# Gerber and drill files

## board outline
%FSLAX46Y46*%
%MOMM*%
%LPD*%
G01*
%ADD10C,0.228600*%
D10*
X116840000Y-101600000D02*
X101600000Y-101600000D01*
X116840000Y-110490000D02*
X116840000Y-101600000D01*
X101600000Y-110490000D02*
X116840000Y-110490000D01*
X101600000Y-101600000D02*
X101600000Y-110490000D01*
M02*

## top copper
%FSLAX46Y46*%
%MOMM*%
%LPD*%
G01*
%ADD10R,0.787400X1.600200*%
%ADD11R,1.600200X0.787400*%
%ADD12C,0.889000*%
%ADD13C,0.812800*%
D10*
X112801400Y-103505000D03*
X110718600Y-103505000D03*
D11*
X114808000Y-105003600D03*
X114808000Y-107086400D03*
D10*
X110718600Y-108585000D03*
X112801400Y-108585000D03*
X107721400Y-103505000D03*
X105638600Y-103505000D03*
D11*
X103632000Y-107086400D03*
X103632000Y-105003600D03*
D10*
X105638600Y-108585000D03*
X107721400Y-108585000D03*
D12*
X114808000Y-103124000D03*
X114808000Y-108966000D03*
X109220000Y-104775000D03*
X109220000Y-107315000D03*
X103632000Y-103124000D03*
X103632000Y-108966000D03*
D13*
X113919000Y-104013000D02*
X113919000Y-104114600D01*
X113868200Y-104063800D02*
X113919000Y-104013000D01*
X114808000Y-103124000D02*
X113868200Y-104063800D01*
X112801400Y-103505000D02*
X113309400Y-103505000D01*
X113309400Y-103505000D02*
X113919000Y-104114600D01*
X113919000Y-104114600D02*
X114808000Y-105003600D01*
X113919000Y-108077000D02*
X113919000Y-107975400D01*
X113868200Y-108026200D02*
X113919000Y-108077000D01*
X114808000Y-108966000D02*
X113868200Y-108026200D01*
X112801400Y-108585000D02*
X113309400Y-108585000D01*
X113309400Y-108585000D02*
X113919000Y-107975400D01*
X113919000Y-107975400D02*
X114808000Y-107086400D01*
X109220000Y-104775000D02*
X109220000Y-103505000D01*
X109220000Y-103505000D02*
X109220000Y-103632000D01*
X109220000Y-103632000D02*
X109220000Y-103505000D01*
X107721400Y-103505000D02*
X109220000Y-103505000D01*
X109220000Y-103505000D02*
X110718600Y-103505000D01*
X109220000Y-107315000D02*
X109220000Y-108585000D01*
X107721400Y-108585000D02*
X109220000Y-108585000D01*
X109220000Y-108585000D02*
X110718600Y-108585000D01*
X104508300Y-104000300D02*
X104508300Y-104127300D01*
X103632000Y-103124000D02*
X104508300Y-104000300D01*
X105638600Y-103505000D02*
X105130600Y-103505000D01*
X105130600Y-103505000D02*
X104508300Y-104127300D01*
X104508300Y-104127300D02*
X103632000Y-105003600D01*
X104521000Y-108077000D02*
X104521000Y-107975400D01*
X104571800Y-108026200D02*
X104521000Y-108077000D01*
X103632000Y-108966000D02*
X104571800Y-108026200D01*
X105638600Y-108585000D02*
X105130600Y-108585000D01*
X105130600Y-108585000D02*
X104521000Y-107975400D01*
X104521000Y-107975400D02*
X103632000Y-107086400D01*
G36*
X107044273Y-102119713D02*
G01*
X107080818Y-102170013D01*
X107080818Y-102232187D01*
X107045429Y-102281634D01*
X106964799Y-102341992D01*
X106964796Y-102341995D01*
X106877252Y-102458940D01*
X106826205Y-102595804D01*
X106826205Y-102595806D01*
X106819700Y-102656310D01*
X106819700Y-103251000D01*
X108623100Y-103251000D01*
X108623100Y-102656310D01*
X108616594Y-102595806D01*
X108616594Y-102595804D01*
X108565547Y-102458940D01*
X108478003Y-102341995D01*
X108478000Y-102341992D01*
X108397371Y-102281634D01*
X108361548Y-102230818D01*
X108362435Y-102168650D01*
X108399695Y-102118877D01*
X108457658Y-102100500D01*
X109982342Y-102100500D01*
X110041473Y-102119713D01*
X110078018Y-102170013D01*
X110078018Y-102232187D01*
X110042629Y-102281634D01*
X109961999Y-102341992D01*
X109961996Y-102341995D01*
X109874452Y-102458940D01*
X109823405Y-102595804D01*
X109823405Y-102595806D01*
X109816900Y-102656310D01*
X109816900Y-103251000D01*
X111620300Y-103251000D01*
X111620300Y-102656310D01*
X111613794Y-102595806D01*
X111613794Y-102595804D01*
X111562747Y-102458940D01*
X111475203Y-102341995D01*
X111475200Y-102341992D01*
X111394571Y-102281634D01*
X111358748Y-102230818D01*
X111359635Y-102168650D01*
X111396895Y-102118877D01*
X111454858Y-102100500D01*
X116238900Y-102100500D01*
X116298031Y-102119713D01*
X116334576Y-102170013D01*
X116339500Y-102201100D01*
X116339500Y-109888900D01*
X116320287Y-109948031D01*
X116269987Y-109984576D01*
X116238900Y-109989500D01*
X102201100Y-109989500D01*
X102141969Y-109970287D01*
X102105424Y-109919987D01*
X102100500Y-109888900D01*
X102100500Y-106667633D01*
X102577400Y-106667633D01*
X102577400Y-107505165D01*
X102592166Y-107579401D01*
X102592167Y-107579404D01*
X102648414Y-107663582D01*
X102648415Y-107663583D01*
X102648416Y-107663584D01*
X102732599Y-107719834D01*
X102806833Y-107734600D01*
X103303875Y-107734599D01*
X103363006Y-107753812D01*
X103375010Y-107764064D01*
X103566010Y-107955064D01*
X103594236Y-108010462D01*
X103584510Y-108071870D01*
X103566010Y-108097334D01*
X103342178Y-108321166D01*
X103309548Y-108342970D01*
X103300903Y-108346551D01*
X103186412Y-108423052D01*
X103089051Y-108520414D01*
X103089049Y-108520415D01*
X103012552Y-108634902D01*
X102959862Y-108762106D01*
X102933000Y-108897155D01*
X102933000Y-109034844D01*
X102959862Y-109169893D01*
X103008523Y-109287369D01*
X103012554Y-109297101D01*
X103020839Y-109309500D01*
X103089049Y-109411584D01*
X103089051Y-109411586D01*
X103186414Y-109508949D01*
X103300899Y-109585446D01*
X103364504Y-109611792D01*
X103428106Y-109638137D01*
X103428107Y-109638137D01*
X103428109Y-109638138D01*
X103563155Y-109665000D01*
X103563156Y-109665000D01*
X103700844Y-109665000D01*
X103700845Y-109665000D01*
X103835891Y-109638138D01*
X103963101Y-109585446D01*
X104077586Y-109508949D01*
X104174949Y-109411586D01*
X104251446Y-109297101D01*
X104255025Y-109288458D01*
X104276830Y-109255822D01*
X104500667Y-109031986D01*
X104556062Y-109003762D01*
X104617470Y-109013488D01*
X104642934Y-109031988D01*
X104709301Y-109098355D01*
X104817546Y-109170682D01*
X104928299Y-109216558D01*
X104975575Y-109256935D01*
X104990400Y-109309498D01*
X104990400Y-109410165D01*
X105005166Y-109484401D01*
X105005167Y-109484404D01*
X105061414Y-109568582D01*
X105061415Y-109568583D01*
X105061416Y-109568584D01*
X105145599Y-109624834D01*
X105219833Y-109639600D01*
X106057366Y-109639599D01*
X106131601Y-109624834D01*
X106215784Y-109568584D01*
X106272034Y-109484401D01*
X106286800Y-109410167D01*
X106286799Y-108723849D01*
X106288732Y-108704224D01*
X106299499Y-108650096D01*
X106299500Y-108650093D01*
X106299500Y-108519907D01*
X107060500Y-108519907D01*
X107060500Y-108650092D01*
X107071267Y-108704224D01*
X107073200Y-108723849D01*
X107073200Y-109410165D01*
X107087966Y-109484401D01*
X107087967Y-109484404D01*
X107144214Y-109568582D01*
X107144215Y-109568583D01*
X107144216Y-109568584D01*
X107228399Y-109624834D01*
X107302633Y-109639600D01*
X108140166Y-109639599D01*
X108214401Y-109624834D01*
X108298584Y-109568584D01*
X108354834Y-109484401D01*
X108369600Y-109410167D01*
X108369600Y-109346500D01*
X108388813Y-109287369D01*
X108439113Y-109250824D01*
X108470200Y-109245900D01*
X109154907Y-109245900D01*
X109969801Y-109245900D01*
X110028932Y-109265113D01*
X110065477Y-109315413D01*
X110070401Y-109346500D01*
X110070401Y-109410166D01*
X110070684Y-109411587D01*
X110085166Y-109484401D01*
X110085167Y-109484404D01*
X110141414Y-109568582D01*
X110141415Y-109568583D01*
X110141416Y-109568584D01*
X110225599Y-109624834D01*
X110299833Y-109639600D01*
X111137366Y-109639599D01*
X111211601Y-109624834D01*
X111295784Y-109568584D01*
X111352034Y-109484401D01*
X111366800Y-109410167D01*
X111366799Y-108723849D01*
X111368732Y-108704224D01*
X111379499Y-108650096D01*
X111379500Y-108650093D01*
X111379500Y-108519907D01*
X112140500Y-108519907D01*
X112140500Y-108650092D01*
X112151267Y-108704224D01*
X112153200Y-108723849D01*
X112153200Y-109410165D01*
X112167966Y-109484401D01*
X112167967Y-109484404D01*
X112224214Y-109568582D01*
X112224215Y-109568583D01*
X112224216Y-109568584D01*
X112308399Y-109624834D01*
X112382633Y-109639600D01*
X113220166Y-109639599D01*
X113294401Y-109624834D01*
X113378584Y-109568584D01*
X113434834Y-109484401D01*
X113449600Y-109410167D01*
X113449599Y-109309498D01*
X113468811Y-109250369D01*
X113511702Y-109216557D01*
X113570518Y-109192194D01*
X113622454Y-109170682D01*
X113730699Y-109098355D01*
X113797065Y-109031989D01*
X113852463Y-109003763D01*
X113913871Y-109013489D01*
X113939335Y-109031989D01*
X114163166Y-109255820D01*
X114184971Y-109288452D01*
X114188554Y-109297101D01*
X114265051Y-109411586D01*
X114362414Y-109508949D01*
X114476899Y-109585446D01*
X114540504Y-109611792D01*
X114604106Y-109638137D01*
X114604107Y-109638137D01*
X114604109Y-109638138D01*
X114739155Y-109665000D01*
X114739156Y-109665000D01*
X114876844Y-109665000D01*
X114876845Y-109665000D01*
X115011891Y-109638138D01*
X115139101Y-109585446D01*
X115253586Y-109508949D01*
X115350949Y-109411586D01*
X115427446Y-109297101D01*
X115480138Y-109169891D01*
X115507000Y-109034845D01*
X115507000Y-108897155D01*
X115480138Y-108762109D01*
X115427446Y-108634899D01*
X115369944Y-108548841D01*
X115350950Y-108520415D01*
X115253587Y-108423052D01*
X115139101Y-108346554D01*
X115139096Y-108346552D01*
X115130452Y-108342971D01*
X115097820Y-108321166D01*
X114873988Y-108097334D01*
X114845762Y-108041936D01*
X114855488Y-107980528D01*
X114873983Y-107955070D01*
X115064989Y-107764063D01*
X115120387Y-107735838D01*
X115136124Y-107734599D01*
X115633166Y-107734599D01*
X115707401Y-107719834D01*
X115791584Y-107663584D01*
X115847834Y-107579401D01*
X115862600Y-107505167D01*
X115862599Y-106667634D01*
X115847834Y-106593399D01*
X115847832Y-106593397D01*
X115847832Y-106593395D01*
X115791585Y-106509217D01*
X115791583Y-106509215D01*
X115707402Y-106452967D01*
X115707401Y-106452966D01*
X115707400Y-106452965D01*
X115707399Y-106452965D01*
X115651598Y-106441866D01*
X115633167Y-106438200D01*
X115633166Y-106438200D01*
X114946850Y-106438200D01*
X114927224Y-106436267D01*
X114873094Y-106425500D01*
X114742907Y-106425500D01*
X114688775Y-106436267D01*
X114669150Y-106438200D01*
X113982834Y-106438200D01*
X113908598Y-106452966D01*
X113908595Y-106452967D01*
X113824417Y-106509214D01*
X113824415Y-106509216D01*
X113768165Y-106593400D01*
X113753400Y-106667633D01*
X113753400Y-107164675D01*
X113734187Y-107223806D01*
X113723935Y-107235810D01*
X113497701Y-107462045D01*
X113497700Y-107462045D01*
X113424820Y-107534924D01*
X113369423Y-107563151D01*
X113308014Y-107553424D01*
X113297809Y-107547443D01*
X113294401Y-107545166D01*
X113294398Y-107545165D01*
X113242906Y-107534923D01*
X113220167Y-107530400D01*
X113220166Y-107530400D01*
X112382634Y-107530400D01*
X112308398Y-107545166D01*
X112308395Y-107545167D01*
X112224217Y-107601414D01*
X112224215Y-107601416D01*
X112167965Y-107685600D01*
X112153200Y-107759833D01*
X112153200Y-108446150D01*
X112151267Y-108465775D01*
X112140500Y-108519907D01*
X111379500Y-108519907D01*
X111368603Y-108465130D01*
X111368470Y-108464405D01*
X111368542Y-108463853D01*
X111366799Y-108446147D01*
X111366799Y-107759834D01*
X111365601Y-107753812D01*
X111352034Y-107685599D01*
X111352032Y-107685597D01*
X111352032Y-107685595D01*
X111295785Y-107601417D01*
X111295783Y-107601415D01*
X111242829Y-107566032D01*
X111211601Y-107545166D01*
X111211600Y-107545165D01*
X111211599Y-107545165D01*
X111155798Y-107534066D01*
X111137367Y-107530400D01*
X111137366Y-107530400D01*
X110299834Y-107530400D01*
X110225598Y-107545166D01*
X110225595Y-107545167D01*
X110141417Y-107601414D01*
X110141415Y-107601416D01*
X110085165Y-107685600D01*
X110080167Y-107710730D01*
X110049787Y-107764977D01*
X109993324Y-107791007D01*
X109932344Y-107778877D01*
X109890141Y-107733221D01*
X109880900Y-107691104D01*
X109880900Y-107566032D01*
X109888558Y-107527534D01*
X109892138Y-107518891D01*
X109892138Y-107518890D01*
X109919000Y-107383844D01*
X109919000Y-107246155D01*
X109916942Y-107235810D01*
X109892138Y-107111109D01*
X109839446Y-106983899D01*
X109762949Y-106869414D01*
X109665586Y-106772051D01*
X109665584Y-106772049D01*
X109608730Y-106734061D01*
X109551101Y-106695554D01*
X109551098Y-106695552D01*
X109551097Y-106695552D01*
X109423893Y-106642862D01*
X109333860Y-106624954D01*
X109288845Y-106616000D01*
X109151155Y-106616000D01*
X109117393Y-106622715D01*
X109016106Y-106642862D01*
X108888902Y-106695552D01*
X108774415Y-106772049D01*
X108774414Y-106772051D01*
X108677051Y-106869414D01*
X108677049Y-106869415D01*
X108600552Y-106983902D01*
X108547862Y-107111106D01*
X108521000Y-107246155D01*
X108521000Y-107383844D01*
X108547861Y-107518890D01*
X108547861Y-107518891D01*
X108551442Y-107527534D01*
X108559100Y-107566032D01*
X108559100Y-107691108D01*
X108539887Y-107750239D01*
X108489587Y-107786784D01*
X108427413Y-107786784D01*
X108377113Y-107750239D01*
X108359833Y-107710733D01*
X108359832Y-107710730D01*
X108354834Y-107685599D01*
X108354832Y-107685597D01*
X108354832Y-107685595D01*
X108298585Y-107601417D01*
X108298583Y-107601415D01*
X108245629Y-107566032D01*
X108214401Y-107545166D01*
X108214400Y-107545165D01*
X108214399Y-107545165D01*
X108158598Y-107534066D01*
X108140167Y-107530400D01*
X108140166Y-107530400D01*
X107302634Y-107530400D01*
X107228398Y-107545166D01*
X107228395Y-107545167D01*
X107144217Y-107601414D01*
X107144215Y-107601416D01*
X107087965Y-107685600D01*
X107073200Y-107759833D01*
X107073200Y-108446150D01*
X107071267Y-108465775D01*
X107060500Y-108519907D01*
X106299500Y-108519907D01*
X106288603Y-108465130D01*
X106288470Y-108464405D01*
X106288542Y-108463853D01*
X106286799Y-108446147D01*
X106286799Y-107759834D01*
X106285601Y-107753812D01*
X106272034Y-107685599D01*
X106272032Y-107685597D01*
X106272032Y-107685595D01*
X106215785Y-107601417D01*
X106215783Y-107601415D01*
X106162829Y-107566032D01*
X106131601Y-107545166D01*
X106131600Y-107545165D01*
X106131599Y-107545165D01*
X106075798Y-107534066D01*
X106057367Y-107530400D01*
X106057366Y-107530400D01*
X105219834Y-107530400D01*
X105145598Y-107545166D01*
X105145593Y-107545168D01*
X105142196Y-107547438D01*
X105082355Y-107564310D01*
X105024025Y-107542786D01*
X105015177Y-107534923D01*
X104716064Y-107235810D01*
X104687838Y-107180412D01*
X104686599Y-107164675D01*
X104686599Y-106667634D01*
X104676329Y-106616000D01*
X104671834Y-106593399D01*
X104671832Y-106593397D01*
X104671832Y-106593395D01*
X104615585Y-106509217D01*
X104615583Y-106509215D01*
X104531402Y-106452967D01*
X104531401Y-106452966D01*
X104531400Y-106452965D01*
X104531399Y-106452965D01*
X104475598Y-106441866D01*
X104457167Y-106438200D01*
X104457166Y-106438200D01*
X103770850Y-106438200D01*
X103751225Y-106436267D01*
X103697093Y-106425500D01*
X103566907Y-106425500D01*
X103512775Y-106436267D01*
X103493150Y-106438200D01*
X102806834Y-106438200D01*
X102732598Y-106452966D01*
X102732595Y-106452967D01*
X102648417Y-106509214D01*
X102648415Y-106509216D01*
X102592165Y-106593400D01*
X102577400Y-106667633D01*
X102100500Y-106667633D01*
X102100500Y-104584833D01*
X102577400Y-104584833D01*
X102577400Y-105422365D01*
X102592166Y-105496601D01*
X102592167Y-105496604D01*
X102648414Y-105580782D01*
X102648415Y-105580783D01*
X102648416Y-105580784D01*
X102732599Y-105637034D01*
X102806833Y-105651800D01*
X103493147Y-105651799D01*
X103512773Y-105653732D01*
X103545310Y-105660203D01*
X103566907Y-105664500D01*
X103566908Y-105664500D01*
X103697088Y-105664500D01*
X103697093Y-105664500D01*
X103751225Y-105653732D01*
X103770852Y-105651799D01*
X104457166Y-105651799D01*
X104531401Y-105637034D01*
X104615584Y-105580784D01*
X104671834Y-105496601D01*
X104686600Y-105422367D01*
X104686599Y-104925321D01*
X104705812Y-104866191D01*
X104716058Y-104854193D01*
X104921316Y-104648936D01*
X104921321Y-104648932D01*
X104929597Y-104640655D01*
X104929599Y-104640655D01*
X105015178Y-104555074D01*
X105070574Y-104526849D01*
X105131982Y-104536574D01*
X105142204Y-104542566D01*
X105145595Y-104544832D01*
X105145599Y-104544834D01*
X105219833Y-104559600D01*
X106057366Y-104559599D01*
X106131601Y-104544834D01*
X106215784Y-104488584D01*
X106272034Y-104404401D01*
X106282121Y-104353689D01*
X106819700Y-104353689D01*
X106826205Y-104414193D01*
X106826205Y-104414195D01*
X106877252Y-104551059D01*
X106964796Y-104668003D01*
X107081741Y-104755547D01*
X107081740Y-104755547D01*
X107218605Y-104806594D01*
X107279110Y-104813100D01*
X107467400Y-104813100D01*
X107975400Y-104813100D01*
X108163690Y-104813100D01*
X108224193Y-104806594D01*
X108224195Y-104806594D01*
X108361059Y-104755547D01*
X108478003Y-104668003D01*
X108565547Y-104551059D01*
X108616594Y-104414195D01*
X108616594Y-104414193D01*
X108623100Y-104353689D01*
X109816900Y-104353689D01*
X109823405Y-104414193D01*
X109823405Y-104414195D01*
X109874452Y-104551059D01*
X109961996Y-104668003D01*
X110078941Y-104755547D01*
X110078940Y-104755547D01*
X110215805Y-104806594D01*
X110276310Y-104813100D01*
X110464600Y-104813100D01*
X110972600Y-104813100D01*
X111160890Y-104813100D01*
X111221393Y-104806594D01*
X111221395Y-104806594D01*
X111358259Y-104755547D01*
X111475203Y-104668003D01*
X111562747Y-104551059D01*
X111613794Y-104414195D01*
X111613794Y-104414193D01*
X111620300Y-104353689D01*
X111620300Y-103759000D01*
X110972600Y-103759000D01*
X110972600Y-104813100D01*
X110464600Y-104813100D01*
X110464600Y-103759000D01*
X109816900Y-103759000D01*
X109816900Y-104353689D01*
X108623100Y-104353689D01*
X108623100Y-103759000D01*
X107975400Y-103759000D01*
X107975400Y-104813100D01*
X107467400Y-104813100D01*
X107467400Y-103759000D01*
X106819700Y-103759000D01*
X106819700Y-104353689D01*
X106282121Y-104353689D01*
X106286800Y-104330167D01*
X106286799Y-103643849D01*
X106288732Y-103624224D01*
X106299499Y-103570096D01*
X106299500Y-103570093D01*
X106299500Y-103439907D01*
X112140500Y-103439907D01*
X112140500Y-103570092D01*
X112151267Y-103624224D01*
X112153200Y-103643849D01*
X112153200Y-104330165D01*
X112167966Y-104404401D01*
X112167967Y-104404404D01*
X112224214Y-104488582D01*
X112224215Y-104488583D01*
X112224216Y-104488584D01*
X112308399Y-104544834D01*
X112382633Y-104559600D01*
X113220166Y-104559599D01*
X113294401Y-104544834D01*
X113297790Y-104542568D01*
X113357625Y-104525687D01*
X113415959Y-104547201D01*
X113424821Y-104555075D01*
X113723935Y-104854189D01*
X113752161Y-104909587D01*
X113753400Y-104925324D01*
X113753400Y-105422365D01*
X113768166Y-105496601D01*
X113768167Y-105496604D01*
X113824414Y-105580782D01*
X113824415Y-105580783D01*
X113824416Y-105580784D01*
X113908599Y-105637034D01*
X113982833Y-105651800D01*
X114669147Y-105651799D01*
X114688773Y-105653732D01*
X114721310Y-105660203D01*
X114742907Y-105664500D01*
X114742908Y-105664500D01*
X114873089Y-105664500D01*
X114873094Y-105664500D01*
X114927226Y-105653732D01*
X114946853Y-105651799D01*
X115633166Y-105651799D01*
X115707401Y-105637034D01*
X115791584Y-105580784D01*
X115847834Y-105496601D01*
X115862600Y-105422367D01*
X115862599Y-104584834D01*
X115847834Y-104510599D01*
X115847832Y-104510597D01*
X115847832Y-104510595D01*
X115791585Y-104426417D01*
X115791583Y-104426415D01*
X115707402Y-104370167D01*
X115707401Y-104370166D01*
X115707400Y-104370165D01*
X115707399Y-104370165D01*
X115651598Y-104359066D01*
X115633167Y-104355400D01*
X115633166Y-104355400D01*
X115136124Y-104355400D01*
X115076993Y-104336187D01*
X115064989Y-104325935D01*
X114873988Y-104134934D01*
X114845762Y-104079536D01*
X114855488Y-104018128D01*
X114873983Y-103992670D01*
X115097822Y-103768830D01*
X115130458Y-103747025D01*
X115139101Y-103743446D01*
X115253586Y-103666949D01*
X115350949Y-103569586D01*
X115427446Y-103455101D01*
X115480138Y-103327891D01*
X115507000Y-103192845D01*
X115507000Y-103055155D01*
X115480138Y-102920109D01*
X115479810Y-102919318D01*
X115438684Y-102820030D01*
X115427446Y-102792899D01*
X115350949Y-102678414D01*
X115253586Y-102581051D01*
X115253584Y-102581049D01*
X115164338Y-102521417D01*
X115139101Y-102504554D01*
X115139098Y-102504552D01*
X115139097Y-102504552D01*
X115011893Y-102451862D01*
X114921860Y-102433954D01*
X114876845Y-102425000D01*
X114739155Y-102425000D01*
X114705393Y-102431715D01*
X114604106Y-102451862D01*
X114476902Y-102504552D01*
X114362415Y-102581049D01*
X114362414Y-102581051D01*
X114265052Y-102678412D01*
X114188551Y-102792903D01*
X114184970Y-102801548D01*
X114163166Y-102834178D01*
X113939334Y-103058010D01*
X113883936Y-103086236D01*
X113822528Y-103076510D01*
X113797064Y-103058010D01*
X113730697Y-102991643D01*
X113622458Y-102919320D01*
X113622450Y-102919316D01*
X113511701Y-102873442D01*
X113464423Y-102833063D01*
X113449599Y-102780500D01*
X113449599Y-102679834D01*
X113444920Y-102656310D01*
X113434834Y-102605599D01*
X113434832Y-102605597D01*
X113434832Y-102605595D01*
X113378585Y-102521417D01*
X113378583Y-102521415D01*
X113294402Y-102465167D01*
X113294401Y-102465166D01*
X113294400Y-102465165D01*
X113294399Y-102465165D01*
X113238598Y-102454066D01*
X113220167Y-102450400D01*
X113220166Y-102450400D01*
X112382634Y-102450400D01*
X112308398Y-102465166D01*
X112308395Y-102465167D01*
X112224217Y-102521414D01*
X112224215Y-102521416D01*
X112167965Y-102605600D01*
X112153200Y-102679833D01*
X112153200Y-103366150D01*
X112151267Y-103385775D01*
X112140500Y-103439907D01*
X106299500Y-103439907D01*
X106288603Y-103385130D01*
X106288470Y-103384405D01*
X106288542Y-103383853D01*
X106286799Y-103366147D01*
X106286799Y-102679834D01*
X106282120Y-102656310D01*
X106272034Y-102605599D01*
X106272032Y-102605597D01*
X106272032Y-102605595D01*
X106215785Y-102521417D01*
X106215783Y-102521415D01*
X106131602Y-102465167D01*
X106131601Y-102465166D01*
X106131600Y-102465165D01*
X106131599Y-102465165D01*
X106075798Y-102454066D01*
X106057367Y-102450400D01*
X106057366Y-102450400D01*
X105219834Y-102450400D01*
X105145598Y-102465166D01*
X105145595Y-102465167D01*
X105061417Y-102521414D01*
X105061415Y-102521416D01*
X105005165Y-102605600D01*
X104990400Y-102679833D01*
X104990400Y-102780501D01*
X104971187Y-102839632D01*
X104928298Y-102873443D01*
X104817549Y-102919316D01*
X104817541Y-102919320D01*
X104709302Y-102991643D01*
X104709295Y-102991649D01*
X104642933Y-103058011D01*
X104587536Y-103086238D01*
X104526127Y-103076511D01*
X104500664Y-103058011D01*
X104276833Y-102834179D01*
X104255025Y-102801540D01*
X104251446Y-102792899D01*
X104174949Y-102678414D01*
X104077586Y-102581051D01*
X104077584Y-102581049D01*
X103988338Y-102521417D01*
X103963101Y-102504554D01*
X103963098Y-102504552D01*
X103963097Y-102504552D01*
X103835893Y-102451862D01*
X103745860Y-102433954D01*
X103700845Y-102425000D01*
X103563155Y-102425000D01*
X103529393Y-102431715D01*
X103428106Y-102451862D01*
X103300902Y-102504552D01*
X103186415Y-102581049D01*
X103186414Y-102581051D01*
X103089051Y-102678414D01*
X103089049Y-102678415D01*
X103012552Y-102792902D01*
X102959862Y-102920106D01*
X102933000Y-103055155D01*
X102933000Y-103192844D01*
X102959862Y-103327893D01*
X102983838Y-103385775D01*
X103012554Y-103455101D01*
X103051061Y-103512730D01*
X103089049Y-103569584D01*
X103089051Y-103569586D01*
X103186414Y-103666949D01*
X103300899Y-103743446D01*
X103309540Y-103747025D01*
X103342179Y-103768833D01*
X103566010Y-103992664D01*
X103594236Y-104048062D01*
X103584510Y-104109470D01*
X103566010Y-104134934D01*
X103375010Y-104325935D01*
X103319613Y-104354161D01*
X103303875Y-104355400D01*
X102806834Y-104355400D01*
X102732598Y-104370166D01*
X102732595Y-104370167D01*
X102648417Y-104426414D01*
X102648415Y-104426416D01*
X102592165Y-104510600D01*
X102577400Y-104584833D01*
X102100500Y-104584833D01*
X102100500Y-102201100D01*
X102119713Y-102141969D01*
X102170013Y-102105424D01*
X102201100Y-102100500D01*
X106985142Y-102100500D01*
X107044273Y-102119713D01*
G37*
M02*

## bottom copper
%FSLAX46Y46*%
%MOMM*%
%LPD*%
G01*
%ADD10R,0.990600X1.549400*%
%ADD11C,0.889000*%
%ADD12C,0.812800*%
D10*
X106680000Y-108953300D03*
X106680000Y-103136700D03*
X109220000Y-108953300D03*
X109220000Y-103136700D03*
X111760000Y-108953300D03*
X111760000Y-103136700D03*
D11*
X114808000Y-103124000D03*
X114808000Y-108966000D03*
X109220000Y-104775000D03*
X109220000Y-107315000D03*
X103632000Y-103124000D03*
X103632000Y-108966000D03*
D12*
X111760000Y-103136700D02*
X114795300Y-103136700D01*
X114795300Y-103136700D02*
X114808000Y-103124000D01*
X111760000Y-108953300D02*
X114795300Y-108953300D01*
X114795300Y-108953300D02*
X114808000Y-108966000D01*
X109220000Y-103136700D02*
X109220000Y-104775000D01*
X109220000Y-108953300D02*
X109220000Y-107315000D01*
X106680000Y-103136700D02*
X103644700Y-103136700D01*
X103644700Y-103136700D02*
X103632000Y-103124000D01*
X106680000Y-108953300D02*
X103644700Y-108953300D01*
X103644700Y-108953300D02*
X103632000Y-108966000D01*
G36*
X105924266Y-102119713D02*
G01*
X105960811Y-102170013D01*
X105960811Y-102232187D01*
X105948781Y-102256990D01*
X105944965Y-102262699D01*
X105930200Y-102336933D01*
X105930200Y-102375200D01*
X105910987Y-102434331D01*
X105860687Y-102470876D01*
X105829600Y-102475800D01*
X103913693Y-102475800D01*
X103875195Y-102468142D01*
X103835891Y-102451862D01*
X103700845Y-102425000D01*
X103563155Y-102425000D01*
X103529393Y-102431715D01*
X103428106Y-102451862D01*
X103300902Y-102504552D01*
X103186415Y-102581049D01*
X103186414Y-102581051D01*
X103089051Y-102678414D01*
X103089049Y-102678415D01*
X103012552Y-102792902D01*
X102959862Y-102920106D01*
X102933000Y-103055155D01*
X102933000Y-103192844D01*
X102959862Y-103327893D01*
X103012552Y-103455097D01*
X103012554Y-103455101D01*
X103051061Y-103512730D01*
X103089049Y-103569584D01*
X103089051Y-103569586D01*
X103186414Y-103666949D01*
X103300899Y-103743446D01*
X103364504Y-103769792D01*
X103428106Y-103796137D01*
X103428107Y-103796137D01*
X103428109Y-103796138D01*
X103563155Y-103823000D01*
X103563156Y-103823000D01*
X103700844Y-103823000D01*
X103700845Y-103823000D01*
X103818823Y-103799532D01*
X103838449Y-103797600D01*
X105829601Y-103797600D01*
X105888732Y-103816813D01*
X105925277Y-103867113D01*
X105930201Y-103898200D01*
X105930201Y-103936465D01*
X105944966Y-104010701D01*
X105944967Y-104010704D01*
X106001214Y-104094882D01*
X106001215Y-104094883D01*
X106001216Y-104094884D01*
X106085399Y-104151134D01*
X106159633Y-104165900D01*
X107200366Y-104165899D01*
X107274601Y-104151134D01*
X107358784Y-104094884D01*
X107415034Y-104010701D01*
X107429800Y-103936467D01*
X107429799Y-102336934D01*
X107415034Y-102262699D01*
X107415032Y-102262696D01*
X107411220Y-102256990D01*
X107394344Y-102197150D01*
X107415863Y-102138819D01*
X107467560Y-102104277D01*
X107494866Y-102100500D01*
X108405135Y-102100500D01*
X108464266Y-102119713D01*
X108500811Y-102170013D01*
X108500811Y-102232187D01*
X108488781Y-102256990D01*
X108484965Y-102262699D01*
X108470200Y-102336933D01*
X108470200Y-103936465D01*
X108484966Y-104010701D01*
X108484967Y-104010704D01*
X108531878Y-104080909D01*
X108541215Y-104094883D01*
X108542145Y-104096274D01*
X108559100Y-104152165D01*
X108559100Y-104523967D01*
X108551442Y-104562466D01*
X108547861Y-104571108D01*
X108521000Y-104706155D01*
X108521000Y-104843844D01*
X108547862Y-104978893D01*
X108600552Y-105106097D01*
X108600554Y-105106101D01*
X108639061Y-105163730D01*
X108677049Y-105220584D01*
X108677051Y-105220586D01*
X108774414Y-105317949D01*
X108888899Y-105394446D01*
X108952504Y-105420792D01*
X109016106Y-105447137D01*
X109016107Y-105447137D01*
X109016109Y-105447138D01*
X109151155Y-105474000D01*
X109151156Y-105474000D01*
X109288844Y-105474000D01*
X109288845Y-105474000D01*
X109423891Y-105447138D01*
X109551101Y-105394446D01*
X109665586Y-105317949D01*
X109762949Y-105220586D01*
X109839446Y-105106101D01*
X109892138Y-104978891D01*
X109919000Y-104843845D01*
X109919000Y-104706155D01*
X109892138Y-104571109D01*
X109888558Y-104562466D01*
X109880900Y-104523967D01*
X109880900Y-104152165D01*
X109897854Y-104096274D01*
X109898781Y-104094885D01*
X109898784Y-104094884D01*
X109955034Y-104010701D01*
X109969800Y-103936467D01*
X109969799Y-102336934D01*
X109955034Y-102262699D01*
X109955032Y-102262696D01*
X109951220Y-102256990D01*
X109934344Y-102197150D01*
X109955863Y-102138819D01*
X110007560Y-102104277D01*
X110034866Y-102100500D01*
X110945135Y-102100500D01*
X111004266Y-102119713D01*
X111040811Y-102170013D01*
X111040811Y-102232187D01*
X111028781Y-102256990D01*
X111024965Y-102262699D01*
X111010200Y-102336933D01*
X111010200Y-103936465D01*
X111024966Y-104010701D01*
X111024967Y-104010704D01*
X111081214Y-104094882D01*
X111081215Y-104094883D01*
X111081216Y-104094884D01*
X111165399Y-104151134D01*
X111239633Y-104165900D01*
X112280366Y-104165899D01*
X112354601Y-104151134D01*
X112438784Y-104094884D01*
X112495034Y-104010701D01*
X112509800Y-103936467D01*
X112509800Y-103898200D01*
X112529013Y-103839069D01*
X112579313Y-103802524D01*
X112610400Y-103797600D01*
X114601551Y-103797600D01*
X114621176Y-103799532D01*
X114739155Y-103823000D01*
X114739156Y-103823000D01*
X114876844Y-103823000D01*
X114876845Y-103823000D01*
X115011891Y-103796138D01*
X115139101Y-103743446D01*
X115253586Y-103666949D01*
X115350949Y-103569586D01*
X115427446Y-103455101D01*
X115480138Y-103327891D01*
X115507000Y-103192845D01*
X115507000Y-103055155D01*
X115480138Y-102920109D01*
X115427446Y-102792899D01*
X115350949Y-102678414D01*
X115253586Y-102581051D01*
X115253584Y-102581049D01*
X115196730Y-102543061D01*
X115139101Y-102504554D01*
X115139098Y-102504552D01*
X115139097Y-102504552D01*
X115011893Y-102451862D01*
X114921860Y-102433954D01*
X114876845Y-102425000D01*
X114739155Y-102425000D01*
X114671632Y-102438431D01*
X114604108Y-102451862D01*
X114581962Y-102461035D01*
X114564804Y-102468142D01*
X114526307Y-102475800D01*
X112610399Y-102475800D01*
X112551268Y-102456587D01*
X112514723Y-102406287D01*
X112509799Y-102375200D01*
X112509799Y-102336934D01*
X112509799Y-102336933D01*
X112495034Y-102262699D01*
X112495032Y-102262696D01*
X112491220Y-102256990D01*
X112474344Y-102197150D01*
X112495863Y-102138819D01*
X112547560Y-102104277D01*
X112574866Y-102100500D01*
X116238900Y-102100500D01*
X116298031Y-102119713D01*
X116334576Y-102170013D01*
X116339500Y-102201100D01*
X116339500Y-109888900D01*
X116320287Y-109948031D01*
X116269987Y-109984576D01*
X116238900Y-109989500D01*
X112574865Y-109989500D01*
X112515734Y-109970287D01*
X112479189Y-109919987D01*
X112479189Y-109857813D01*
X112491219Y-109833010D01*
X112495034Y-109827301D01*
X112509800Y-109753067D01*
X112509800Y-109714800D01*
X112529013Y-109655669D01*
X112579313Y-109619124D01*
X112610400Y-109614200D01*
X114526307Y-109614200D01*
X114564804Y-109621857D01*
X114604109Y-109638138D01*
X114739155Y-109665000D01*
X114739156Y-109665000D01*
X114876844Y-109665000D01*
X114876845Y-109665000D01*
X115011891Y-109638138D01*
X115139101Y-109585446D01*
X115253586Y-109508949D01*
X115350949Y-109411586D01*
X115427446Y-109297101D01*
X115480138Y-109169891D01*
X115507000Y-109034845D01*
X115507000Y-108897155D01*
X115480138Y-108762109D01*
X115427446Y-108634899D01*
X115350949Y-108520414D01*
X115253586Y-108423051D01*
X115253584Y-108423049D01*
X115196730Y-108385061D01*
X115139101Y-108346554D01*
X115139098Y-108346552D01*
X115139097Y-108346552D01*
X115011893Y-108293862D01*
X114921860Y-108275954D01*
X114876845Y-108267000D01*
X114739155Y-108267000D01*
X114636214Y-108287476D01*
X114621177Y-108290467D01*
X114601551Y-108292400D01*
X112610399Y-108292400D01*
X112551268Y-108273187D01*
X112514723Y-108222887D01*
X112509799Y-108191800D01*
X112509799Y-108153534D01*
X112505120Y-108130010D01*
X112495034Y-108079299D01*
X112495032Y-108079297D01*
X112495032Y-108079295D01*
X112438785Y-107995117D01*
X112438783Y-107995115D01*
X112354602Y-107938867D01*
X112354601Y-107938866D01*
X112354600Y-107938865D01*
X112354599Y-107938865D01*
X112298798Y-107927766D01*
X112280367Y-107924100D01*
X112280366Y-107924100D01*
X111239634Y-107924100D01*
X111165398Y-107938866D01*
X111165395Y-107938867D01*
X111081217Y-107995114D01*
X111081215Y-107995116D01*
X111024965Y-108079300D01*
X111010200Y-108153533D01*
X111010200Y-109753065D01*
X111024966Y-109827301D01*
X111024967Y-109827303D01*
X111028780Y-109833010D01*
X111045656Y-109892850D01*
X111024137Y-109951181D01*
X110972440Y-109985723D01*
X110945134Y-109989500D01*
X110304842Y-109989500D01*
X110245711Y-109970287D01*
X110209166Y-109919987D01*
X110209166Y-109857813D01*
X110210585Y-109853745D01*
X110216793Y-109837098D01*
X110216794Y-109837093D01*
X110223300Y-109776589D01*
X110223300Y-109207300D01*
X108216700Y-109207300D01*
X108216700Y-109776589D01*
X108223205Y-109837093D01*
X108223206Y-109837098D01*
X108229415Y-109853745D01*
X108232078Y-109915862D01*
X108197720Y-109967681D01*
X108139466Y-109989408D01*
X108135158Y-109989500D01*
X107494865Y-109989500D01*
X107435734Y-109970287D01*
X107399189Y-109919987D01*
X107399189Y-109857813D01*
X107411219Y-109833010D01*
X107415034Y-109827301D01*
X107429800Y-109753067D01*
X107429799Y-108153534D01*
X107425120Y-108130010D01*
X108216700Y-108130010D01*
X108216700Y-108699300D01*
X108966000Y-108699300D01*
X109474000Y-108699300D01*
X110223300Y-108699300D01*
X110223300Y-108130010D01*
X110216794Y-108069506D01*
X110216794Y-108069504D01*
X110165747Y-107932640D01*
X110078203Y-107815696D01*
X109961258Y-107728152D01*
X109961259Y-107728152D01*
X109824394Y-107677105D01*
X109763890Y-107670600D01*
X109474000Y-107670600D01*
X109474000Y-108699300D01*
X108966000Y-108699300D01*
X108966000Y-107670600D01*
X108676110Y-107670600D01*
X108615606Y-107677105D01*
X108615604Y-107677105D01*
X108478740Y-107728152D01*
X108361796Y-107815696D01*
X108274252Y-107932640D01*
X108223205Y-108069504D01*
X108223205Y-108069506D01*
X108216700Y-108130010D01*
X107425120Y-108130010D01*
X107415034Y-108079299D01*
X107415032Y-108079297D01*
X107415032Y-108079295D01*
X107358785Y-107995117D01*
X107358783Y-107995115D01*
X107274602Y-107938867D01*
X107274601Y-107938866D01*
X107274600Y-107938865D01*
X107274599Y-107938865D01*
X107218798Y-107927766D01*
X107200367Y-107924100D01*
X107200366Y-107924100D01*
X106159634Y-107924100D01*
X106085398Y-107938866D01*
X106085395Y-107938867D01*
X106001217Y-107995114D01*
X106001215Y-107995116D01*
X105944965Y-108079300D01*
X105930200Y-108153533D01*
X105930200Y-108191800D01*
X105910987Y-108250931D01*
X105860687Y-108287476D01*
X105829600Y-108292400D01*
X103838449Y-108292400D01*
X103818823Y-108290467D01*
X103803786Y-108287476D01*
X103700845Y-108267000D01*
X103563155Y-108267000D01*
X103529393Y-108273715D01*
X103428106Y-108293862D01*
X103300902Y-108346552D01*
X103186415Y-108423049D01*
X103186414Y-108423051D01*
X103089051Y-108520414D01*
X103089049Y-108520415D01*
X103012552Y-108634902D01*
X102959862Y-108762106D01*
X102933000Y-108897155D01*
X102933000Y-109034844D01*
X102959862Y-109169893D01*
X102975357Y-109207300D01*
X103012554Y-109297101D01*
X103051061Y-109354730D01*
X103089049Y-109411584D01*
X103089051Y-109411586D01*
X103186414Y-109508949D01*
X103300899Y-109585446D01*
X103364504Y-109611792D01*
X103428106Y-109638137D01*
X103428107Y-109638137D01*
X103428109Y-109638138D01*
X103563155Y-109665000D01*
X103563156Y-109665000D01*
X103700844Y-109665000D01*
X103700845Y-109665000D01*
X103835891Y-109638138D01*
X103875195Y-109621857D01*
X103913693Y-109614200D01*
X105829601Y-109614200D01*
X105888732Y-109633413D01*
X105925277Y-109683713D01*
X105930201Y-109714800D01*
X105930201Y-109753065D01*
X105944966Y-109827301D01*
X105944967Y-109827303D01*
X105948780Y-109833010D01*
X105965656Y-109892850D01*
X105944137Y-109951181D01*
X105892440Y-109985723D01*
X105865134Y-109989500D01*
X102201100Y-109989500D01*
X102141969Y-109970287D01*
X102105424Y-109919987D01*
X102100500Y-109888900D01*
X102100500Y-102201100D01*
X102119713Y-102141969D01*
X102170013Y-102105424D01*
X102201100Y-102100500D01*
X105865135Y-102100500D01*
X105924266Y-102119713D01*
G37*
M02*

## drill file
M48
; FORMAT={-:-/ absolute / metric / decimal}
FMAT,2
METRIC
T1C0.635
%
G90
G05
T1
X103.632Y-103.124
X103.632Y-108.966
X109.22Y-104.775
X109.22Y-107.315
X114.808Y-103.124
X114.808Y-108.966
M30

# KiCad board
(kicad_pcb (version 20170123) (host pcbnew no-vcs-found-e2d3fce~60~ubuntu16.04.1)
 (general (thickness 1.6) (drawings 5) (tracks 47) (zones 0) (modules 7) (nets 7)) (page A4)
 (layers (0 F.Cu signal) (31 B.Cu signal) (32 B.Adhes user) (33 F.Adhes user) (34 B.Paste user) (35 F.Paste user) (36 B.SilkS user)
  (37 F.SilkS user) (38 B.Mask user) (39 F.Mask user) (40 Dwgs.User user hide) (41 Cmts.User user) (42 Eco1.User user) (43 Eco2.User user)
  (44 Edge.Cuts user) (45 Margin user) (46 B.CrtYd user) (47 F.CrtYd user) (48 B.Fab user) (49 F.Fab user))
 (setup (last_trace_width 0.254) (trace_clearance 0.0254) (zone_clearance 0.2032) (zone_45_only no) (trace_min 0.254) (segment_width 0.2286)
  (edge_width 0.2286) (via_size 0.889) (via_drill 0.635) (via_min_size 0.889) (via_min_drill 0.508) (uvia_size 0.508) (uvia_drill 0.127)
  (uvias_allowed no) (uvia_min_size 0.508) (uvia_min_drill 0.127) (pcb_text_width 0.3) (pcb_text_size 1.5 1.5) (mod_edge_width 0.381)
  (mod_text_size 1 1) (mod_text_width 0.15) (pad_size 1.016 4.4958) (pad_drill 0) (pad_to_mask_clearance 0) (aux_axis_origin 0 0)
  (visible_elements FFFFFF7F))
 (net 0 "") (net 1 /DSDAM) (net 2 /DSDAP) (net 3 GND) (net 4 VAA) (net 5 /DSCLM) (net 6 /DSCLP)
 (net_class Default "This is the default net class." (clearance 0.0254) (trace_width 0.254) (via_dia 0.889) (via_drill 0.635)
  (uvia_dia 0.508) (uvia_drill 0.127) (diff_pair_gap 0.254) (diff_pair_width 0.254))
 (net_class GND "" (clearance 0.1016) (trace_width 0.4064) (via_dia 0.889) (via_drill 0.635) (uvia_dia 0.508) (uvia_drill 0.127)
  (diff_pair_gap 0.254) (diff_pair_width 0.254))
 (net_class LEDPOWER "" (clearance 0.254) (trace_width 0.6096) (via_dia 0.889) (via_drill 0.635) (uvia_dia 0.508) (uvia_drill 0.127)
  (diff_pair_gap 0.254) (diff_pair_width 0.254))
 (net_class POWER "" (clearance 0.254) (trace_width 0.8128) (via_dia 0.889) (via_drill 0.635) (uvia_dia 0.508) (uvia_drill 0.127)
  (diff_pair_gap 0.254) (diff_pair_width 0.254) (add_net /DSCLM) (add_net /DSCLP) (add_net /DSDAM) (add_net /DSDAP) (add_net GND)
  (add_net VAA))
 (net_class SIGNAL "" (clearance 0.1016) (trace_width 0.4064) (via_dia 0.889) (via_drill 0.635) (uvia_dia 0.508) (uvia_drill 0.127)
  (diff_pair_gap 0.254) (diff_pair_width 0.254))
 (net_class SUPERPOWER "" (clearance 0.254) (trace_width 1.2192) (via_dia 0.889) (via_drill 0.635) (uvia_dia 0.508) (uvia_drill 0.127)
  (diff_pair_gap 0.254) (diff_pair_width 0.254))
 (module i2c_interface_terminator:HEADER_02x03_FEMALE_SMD (layer B.Cu) (at 109.22 106.045 180)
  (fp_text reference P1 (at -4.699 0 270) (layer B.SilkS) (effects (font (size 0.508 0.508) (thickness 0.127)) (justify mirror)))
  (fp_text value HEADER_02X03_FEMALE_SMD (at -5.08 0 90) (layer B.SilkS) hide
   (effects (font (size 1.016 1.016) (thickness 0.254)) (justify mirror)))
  (pad 6 smd rect (at 2.54 -2.9083 180) (size 0.9906 1.5494) (layers B.Cu B.Paste B.Mask) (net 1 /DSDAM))
  (pad 5 smd rect (at 2.54 2.9083 180) (size 0.9906 1.5494) (layers B.Cu B.Paste B.Mask) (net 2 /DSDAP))
  (pad 4 smd rect (at 0 -2.9083 180) (size 0.9906 1.5494) (layers B.Cu B.Paste B.Mask) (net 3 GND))
  (pad 3 smd rect (at 0 2.9083 180) (size 0.9906 1.5494) (layers B.Cu B.Paste B.Mask) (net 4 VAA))
  (pad 2 smd rect (at -2.54 -2.9083 180) (size 0.9906 1.5494) (layers B.Cu B.Paste B.Mask) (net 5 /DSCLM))
  (pad 1 smd rect (at -2.54 2.9083 180) (size 0.9906 1.5494) (layers B.Cu B.Paste B.Mask) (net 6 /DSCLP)))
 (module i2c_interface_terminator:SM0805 (layer F.Cu) (at 111.76 103.505)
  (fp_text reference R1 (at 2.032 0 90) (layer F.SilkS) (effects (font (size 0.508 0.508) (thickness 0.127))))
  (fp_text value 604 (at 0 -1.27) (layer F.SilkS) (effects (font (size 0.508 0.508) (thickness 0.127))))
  (pad 2 smd rect (at 1.0414 0) (size 0.7874 1.6002) (layers F.Cu F.Paste F.Mask) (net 6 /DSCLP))
  (pad 1 smd rect (at -1.0414 0) (size 0.7874 1.6002) (layers F.Cu F.Paste F.Mask) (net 4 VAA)))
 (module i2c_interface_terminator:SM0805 (layer F.Cu) (at 114.808 106.045 270)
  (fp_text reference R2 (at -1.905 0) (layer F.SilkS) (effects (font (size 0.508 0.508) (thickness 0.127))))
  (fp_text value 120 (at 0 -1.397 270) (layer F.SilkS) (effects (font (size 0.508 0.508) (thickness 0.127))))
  (pad 1 smd rect (at -1.0414 0 270) (size 0.7874 1.6002) (layers F.Cu F.Paste F.Mask) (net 6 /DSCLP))
  (pad 2 smd rect (at 1.0414 0 270) (size 0.7874 1.6002) (layers F.Cu F.Paste F.Mask) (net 5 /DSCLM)))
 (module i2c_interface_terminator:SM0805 (layer F.Cu) (at 111.76 108.585 180)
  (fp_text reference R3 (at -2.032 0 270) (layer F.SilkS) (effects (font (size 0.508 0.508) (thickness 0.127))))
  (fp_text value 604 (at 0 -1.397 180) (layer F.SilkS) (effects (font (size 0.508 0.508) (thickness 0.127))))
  (pad 2 smd rect (at 1.0414 0 180) (size 0.7874 1.6002) (layers F.Cu F.Paste F.Mask) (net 3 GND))
  (pad 1 smd rect (at -1.0414 0 180) (size 0.7874 1.6002) (layers F.Cu F.Paste F.Mask) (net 5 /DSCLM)))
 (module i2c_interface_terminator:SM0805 (layer F.Cu) (at 106.68 103.505 180)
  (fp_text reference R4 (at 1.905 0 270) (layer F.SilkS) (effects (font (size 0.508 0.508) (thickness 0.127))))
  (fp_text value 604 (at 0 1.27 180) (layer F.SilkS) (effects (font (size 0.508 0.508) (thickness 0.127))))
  (pad 1 smd rect (at -1.0414 0 180) (size 0.7874 1.6002) (layers F.Cu F.Paste F.Mask) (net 4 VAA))
  (pad 2 smd rect (at 1.0414 0 180) (size 0.7874 1.6002) (layers F.Cu F.Paste F.Mask) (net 2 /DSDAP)))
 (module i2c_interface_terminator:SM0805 (layer F.Cu) (at 103.632 106.045 270)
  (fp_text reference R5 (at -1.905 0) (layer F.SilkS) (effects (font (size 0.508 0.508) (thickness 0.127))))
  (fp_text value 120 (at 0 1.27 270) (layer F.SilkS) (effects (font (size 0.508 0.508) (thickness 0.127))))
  (pad 2 smd rect (at 1.0414 0 270) (size 0.7874 1.6002) (layers F.Cu F.Paste F.Mask) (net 1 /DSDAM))
  (pad 1 smd rect (at -1.0414 0 270) (size 0.7874 1.6002) (layers F.Cu F.Paste F.Mask) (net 2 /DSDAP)))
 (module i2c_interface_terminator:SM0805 (layer F.Cu) (at 106.68 108.585)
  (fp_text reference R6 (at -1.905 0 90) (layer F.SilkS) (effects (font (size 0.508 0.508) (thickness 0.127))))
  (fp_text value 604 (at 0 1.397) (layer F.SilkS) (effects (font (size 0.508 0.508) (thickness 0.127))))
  (pad 1 smd rect (at -1.0414 0) (size 0.7874 1.6002) (layers F.Cu F.Paste F.Mask) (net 1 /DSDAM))
  (pad 2 smd rect (at 1.0414 0) (size 0.7874 1.6002) (layers F.Cu F.Paste F.Mask) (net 3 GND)))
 (gr_line (start 116.84 101.6) (end 101.6 101.6) (angle 90) (layer Edge.Cuts) (width 0.2286))
 (gr_line (start 116.84 110.49) (end 116.84 101.6) (angle 90) (layer Edge.Cuts) (width 0.2286))
 (gr_line (start 101.6 110.49) (end 116.84 110.49) (angle 90) (layer Edge.Cuts) (width 0.2286))
 (gr_line (start 101.6 101.6) (end 101.6 110.49) (angle 90) (layer Edge.Cuts) (width 0.2286))
 (segment (start 111.76 103.1367) (end 114.7953 103.1367) (width 0.8128) (layer B.Cu) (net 6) (status 400000))
 (segment (start 113.919 104.013) (end 113.919 104.1146) (width 0.8128) (layer F.Cu) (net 6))
 (segment (start 113.8682 104.0638) (end 113.919 104.013) (width 0.8128) (layer F.Cu) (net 6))
 (segment (start 114.808 103.124) (end 113.8682 104.0638) (width 0.8128) (layer F.Cu) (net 6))
 (via (at 114.808 103.124) (size 0.889) (drill 0.635) (layers F.Cu B.Cu) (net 6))
 (segment (start 114.7953 103.1367) (end 114.808 103.124) (width 0.8128) (layer B.Cu) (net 6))
 (segment (start 112.8014 103.505) (end 113.3094 103.505) (width 0.8128) (layer F.Cu) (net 6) (status 400000))
 (segment (start 113.3094 103.505) (end 113.919 104.1146) (width 0.8128) (layer F.Cu) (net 6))
 (segment (start 113.919 104.1146) (end 114.808 105.0036) (width 0.8128) (layer F.Cu) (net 6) (status 800000))
 (segment (start 111.76 108.9533) (end 114.7953 108.9533) (width 0.8128) (layer B.Cu) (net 5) (status 400000))
 (segment (start 113.919 108.077) (end 113.919 107.9754) (width 0.8128) (layer F.Cu) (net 5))
 (segment (start 113.8682 108.0262) (end 113.919 108.077) (width 0.8128) (layer F.Cu) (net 5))
 (segment (start 114.808 108.966) (end 113.8682 108.0262) (width 0.8128) (layer F.Cu) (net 5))
 (via (at 114.808 108.966) (size 0.889) (drill 0.635) (layers F.Cu B.Cu) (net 5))
 (segment (start 114.7953 108.9533) (end 114.808 108.966) (width 0.8128) (layer B.Cu) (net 5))
 (segment (start 112.8014 108.585) (end 113.3094 108.585) (width 0.8128) (layer F.Cu) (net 5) (status 400000))
 (segment (start 113.3094 108.585) (end 113.919 107.9754) (width 0.8128) (layer F.Cu) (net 5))
 (segment (start 113.919 107.9754) (end 114.808 107.0864) (width 0.8128) (layer F.Cu) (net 5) (status 800000))
 (segment (start 109.22 103.1367) (end 109.22 104.775) (width 0.8128) (layer B.Cu) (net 4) (status 400000))
 (segment (start 109.22 104.775) (end 109.22 103.505) (width 0.8128) (layer F.Cu) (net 4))
 (via (at 109.22 104.775) (size 0.889) (drill 0.635) (layers F.Cu B.Cu) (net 4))
 (segment (start 109.22 103.505) (end 109.22 103.632) (width 0.8128) (layer F.Cu) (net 4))
 (segment (start 109.22 103.632) (end 109.22 103.505) (width 0.8128) (layer F.Cu) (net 4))
 (segment (start 107.7214 103.505) (end 109.22 103.505) (width 0.8128) (layer F.Cu) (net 4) (status 400000))
 (segment (start 109.22 103.505) (end 110.7186 103.505) (width 0.8128) (layer F.Cu) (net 4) (status 800000))
 (segment (start 109.22 108.9533) (end 109.22 107.315) (width 0.8128) (layer B.Cu) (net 3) (status 400000))
 (segment (start 109.22 107.315) (end 109.22 108.585) (width 0.8128) (layer F.Cu) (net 3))
 (via (at 109.22 107.315) (size 0.889) (drill 0.635) (layers F.Cu B.Cu) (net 3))
 (segment (start 107.7214 108.585) (end 109.22 108.585) (width 0.8128) (layer F.Cu) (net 3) (status 400000))
 (segment (start 109.22 108.585) (end 110.7186 108.585) (width 0.8128) (layer F.Cu) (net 3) (status 800000))
 (segment (start 106.68 103.1367) (end 103.6447 103.1367) (width 0.8128) (layer B.Cu) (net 2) (status 400000))
 (segment (start 104.5083 104.0003) (end 104.5083 104.1273) (width 0.8128) (layer F.Cu) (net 2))
 (segment (start 103.632 103.124) (end 104.5083 104.0003) (width 0.8128) (layer F.Cu) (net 2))
 (via (at 103.632 103.124) (size 0.889) (drill 0.635) (layers F.Cu B.Cu) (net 2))
 (segment (start 103.6447 103.1367) (end 103.632 103.124) (width 0.8128) (layer B.Cu) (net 2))
 (segment (start 105.6386 103.505) (end 105.1306 103.505) (width 0.8128) (layer F.Cu) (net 2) (status 400000))
 (segment (start 105.1306 103.505) (end 104.5083 104.1273) (width 0.8128) (layer F.Cu) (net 2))
 (segment (start 104.5083 104.1273) (end 103.632 105.0036) (width 0.8128) (layer F.Cu) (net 2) (status 800000))
 (segment (start 106.68 108.9533) (end 103.6447 108.9533) (width 0.8128) (layer B.Cu) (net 1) (status 400000))
 (segment (start 104.521 108.077) (end 104.521 107.9754) (width 0.8128) (layer F.Cu) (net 1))
 (segment (start 104.5718 108.0262) (end 104.521 108.077) (width 0.8128) (layer F.Cu) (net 1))
 (segment (start 103.632 108.966) (end 104.5718 108.0262) (width 0.8128) (layer F.Cu) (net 1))
 (via (at 103.632 108.966) (size 0.889) (drill 0.635) (layers F.Cu B.Cu) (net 1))
 (segment (start 103.6447 108.9533) (end 103.632 108.966) (width 0.8128) (layer B.Cu) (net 1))
 (segment (start 105.6386 108.585) (end 105.1306 108.585) (width 0.8128) (layer F.Cu) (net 1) (status 400000))
 (segment (start 105.1306 108.585) (end 104.521 107.9754) (width 0.8128) (layer F.Cu) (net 1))
 (segment (start 104.521 107.9754) (end 103.632 107.0864) (width 0.8128) (layer F.Cu) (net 1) (status 800000))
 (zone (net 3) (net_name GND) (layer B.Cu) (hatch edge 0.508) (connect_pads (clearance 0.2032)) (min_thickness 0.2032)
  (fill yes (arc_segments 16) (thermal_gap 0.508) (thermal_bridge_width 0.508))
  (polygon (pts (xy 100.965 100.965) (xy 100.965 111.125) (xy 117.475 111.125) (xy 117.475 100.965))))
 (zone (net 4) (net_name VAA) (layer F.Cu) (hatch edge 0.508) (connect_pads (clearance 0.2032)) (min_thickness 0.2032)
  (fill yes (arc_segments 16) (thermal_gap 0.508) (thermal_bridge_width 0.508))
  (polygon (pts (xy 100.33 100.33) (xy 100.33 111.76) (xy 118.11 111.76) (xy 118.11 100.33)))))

